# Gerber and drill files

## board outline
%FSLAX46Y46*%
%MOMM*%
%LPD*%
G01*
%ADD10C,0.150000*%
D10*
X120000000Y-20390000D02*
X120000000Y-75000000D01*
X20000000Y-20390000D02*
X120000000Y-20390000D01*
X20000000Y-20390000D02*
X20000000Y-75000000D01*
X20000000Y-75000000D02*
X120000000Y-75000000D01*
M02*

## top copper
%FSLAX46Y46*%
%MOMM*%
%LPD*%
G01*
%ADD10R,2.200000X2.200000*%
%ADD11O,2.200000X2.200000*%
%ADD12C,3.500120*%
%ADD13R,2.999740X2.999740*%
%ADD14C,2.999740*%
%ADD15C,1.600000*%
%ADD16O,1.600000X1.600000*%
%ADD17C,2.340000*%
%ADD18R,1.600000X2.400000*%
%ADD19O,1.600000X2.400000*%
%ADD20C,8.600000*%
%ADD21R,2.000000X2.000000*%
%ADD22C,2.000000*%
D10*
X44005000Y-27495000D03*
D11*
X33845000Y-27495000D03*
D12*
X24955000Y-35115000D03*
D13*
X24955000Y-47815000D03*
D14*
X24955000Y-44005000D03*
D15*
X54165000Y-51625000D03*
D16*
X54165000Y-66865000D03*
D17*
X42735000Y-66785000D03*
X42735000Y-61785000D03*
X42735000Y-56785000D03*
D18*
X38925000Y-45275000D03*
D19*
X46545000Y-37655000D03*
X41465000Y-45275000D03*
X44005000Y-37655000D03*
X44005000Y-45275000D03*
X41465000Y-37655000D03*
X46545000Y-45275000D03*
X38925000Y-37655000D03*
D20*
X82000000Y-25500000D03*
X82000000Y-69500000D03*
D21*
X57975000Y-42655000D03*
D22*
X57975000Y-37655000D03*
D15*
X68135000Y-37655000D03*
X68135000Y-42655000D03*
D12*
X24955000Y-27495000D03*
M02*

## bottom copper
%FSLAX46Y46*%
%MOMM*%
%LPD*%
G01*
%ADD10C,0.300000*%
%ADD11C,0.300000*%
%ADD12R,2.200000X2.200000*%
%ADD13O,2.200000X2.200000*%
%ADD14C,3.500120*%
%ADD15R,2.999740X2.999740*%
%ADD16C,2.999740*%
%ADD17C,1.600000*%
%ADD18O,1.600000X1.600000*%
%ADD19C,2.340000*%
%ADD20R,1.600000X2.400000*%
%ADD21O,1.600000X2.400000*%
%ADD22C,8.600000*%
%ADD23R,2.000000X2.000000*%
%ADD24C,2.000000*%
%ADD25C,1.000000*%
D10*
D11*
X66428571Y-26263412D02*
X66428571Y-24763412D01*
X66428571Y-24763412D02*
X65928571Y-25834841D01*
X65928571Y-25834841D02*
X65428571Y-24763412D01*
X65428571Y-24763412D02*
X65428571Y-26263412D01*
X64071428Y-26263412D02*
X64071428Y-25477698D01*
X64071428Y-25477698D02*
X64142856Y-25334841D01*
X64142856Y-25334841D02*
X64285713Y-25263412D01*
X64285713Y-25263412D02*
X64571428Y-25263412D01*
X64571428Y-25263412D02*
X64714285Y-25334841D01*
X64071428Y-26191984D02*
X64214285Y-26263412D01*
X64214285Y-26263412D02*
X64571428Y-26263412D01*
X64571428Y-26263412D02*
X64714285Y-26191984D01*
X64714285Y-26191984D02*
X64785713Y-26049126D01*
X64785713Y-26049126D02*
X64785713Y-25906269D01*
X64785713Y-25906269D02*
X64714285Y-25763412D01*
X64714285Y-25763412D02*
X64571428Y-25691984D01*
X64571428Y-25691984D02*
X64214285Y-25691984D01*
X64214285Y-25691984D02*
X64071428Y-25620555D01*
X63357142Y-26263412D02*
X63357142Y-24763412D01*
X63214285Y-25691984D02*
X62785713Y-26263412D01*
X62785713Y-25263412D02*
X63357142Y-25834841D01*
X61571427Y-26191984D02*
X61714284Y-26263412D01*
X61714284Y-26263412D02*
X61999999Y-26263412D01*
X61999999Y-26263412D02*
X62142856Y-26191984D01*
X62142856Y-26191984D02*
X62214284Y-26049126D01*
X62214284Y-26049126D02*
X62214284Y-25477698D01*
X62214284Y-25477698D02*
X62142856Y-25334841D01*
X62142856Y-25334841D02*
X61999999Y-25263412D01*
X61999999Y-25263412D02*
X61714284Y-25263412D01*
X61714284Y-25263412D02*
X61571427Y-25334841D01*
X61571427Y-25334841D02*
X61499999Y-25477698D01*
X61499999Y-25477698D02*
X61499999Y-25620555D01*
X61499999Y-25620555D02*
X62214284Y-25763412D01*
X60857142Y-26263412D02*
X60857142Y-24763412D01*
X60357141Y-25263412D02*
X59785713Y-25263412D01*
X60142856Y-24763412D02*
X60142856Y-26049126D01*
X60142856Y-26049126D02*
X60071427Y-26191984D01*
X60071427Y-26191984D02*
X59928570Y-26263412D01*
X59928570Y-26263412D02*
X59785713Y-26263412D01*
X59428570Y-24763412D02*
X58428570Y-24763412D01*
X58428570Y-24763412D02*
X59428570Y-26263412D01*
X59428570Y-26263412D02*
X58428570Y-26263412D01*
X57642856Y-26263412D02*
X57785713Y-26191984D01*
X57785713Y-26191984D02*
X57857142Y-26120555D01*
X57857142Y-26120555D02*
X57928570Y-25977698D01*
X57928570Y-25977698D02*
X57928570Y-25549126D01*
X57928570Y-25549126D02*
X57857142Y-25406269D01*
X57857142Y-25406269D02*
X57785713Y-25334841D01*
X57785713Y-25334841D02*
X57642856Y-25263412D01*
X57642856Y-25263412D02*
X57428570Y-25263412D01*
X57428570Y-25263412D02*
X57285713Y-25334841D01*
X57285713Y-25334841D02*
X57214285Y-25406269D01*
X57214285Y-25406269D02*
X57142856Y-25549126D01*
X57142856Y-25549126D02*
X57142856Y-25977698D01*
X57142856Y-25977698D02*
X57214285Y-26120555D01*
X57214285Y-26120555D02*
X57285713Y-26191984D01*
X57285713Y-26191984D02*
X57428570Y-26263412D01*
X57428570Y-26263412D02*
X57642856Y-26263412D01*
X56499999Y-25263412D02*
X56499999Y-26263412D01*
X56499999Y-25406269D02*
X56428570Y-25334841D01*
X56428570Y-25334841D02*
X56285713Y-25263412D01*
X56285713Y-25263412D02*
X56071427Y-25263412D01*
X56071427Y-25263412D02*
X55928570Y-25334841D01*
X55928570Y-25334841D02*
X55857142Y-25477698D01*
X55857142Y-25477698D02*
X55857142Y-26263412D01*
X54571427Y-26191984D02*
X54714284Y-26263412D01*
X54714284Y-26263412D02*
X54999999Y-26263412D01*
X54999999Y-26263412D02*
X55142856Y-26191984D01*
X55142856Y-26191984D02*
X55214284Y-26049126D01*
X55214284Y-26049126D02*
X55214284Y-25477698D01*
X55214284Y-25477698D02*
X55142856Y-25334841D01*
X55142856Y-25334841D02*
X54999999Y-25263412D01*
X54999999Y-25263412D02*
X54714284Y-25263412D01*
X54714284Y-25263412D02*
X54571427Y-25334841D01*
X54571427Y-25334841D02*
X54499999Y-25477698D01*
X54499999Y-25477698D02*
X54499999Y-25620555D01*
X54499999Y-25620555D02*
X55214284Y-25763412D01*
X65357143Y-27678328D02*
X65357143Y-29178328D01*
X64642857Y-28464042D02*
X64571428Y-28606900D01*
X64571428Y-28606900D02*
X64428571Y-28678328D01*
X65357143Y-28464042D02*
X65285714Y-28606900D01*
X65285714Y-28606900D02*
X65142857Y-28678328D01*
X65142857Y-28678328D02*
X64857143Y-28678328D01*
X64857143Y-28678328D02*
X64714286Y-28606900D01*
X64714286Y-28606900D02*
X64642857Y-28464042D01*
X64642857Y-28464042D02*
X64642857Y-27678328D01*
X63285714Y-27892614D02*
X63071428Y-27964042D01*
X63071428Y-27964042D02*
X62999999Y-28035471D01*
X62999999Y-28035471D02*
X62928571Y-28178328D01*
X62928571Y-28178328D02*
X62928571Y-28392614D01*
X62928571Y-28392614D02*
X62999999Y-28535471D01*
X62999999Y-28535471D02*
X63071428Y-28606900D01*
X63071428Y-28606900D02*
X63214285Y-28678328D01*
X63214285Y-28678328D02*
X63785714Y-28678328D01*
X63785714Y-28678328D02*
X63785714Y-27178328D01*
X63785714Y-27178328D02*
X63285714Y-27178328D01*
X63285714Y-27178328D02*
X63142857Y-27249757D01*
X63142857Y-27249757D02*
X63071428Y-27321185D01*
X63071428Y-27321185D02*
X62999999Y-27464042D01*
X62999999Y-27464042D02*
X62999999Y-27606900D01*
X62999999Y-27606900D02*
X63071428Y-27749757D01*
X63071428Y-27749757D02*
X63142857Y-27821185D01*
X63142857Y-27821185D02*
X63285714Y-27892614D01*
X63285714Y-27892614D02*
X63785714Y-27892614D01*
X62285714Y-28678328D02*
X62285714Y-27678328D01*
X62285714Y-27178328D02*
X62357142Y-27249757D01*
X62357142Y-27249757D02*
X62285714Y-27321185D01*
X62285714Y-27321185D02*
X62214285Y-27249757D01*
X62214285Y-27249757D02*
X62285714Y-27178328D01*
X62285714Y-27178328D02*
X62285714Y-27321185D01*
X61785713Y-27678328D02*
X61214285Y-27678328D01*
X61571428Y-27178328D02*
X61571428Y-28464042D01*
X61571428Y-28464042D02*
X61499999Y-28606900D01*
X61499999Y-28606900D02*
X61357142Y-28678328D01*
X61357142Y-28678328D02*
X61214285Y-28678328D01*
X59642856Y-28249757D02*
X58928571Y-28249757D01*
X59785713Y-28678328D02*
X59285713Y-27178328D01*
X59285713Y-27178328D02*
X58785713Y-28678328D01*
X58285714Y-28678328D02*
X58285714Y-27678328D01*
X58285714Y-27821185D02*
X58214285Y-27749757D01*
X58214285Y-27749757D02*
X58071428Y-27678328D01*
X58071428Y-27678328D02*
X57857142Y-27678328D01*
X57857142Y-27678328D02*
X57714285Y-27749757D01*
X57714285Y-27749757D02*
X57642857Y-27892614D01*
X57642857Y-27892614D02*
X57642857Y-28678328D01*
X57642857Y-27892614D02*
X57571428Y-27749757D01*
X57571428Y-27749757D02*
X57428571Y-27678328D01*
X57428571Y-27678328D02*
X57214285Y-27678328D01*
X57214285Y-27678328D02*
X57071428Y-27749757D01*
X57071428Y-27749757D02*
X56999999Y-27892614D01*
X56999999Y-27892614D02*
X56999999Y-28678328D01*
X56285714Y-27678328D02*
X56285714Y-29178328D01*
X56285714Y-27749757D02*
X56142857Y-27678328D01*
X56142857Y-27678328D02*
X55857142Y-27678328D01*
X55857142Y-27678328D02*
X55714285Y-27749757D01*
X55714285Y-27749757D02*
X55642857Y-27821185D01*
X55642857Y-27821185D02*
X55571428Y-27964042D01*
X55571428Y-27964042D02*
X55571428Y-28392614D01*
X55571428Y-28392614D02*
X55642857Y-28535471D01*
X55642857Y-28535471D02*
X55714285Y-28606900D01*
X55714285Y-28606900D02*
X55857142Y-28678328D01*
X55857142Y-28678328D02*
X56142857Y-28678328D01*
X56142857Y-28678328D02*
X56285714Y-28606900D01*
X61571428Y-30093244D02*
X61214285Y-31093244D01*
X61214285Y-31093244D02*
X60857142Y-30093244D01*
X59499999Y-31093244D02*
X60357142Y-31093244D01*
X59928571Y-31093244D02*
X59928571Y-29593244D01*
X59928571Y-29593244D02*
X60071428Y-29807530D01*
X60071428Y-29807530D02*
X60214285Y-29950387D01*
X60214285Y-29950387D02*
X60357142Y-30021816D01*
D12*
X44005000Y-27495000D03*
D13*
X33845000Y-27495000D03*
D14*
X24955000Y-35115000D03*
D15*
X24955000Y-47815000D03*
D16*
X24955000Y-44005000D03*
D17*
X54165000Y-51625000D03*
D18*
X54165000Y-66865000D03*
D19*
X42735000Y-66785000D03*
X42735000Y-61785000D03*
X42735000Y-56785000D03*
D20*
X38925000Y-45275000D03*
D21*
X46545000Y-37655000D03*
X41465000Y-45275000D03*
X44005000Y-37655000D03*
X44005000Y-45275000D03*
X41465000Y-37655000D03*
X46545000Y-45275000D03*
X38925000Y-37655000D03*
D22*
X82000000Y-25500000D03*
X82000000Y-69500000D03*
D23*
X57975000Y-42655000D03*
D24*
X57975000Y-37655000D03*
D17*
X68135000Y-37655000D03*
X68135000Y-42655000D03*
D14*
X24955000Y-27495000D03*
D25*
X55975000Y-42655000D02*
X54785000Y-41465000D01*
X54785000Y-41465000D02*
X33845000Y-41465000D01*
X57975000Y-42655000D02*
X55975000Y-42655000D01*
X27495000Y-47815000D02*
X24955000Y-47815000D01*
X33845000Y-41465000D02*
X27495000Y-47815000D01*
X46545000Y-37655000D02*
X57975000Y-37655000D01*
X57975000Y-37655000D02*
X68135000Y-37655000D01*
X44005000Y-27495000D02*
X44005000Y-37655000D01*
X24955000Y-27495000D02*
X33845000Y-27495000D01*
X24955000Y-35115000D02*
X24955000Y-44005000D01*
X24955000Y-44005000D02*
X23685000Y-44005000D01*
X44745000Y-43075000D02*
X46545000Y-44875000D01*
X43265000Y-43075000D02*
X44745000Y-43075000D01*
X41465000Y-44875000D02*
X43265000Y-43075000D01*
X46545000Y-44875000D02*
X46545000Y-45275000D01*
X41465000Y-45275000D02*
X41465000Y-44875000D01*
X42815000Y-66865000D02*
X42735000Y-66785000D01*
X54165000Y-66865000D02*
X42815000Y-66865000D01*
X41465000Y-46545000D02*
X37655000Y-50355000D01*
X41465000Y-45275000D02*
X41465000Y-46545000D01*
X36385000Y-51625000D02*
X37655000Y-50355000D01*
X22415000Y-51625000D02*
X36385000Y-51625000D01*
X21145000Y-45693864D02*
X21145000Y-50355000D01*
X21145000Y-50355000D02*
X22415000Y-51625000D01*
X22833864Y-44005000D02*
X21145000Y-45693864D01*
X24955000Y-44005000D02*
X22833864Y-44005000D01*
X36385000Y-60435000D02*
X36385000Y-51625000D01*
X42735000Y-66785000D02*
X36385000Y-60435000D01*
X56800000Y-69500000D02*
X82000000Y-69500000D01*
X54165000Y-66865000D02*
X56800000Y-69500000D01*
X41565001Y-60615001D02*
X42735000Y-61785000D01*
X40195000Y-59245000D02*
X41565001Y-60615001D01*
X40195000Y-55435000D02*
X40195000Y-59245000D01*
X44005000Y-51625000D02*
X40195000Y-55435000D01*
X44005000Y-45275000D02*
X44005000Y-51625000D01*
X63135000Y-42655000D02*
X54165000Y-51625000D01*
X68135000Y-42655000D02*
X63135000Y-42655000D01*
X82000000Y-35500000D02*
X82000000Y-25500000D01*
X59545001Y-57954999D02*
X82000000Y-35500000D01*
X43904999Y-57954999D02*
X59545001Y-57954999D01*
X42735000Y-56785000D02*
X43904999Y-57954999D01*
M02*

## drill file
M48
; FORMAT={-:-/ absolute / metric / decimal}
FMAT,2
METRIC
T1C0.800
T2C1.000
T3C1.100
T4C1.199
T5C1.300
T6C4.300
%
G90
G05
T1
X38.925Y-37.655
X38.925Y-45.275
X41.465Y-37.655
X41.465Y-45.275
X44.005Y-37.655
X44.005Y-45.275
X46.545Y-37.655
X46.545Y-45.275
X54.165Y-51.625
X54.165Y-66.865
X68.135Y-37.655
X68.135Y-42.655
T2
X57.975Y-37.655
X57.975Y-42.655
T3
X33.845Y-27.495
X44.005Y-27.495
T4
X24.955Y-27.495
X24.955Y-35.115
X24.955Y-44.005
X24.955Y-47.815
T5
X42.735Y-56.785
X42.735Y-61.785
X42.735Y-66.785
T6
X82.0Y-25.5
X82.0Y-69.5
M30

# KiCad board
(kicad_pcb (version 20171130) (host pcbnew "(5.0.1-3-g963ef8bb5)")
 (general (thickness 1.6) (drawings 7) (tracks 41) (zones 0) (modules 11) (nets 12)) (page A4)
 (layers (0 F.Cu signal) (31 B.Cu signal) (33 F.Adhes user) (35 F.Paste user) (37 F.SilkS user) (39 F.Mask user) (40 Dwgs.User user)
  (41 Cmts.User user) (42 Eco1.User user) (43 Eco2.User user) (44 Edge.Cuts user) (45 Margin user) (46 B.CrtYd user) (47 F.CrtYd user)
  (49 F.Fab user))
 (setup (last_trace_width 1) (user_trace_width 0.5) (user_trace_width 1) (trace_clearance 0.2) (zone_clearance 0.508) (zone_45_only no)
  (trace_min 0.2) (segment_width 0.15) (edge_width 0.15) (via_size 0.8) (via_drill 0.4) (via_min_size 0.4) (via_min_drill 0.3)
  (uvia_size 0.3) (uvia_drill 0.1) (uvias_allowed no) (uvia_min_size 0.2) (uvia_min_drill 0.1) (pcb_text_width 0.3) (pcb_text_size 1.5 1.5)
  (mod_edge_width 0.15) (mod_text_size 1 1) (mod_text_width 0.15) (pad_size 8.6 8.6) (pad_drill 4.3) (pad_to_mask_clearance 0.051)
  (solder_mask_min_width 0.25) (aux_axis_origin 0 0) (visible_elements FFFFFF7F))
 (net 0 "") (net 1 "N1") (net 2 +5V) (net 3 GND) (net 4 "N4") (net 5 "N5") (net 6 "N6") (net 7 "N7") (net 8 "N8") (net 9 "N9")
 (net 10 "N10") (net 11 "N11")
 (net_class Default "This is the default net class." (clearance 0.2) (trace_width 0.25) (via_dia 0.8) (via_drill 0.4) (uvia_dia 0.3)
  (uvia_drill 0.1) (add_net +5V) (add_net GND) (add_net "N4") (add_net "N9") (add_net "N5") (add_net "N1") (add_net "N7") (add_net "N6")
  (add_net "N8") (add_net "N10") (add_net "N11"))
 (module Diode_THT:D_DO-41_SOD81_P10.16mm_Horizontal (layer F.Cu) (at 44.005 27.495 180)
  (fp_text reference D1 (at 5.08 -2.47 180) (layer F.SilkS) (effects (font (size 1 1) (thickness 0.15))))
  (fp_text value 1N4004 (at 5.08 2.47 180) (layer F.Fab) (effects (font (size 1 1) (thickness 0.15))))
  (pad 1 thru_hole rect (at 0 0 180) (size 2.2 2.2) (drill 1.1) (layers *.Cu *.Mask) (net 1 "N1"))
  (pad 2 thru_hole oval (at 10.16 0 180) (size 2.2 2.2) (drill 1.1) (layers *.Cu *.Mask) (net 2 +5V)))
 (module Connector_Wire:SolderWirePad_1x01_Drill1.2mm (layer F.Cu) (at 24.955 35.115)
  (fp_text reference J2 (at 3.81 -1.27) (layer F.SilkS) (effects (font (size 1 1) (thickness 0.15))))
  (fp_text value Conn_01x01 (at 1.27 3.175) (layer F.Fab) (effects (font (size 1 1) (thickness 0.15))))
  (pad 1 thru_hole circle (at 0 0) (size 3.50012 3.50012) (drill 1.19888) (layers *.Cu *.Mask) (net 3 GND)))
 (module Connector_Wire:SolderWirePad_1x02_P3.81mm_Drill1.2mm (layer F.Cu) (at 24.955 47.815 90)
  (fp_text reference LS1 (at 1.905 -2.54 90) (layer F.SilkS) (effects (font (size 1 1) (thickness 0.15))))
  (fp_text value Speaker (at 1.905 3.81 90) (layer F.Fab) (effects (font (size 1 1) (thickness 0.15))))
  (pad 1 thru_hole rect (at 0 0 90) (size 2.99974 2.99974) (drill 1.19888) (layers *.Cu *.Mask) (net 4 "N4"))
  (pad 2 thru_hole circle (at 3.81 0 90) (size 2.99974 2.99974) (drill 1.19888) (layers *.Cu *.Mask) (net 3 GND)))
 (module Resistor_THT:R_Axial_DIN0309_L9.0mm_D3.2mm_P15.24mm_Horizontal (layer F.Cu) (at 54.165 51.625 270)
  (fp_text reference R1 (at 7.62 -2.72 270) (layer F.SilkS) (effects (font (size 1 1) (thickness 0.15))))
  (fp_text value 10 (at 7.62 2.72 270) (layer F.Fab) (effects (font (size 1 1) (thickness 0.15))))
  (pad 1 thru_hole circle (at 0 0 270) (size 1.6 1.6) (drill 0.8) (layers *.Cu *.Mask) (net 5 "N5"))
  (pad 2 thru_hole oval (at 15.24 0 270) (size 1.6 1.6) (drill 0.8) (layers *.Cu *.Mask) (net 3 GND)))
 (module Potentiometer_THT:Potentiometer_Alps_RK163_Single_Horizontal (layer F.Cu) (at 42.735 56.785 180)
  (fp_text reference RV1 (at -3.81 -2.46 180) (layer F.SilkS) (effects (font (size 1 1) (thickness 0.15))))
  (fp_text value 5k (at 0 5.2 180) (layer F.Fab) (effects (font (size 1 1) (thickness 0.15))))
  (pad 3 thru_hole circle (at 0 -10 180) (size 2.34 2.34) (drill 1.3) (layers *.Cu *.Mask) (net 3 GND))
  (pad 2 thru_hole circle (at 0 -5 180) (size 2.34 2.34) (drill 1.3) (layers *.Cu *.Mask) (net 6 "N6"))
  (pad 1 thru_hole circle (at 0 0 180) (size 2.34 2.34) (drill 1.3) (layers *.Cu *.Mask) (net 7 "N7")))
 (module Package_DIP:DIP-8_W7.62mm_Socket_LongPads (layer F.Cu) (at 38.925 45.275 90)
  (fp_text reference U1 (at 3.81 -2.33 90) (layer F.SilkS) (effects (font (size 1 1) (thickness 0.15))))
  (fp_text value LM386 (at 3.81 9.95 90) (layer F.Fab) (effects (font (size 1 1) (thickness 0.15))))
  (pad 1 thru_hole rect (at 0 0 90) (size 2.4 1.6) (drill 0.8) (layers *.Cu *.Mask) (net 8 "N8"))
  (pad 5 thru_hole oval (at 7.62 7.62 90) (size 2.4 1.6) (drill 0.8) (layers *.Cu *.Mask) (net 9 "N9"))
  (pad 2 thru_hole oval (at 0 2.54 90) (size 2.4 1.6) (drill 0.8) (layers *.Cu *.Mask) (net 3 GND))
  (pad 6 thru_hole oval (at 7.62 5.08 90) (size 2.4 1.6) (drill 0.8) (layers *.Cu *.Mask) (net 1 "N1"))
  (pad 3 thru_hole oval (at 0 5.08 90) (size 2.4 1.6) (drill 0.8) (layers *.Cu *.Mask) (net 6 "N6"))
  (pad 7 thru_hole oval (at 7.62 2.54 90) (size 2.4 1.6) (drill 0.8) (layers *.Cu *.Mask) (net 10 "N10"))
  (pad 4 thru_hole oval (at 0 7.62 90) (size 2.4 1.6) (drill 0.8) (layers *.Cu *.Mask) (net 3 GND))
  (pad 8 thru_hole oval (at 7.62 0 90) (size 2.4 1.6) (drill 0.8) (layers *.Cu *.Mask) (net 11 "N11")))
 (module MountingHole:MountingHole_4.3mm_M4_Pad (layer F.Cu) (at 82 25.5)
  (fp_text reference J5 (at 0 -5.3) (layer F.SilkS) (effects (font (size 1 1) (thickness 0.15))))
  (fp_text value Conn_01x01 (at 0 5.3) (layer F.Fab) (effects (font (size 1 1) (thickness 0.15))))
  (pad 1 thru_hole circle (at 0 0) (size 8.6 8.6) (drill 4.3) (layers *.Cu *.Mask) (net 7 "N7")))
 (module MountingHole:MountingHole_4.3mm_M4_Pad (layer F.Cu) (at 82 69.5)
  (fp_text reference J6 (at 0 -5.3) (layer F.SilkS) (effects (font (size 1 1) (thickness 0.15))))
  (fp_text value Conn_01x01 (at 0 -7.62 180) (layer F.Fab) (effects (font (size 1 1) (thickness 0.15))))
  (pad 1 thru_hole circle (at 0 0) (size 8.6 8.6) (drill 4.3) (layers *.Cu *.Mask) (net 3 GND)))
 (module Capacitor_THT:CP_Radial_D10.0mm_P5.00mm (layer F.Cu) (at 57.975 42.655 90)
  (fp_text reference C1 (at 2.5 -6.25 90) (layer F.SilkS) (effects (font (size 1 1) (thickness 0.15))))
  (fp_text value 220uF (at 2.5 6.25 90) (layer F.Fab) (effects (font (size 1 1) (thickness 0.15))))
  (pad 1 thru_hole rect (at 0 0 90) (size 2 2) (drill 1) (layers *.Cu *.Mask) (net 4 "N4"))
  (pad 2 thru_hole circle (at 5 0 90) (size 2 2) (drill 1) (layers *.Cu *.Mask) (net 9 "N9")))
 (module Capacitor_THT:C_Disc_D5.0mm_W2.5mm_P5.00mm (layer F.Cu) (at 68.135 37.655 270)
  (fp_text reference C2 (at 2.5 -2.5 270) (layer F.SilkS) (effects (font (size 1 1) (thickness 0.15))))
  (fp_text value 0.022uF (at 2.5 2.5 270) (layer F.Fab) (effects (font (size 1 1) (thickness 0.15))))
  (pad 1 thru_hole circle (at 0 0 270) (size 1.6 1.6) (drill 0.8) (layers *.Cu *.Mask) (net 9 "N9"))
  (pad 2 thru_hole circle (at 5 0 270) (size 1.6 1.6) (drill 0.8) (layers *.Cu *.Mask) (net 5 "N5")))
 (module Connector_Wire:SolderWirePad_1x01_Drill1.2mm (layer F.Cu) (at 24.955 27.495)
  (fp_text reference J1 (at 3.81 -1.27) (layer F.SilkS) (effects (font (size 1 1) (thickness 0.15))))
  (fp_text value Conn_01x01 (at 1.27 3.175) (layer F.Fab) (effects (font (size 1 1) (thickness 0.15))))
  (pad 1 thru_hole circle (at 0 0) (size 3.50012 3.50012) (drill 1.19888) (layers *.Cu *.Mask) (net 2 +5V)))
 (gr_line (start 120 20.39) (end 120 75) (layer Edge.Cuts) (width 0.15))
 (gr_line (start 20 20.39) (end 120 20.39) (layer Edge.Cuts) (width 0.15))
 (gr_line (start 20 20.39) (end 20 75) (layer Edge.Cuts) (width 0.15))
 (gr_line (start 20 75) (end 120 75) (layer Edge.Cuts) (width 0.15))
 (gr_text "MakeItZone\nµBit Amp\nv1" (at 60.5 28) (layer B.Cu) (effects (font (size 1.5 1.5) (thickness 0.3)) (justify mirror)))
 (segment (start 55.975 42.655) (end 54.785 41.465) (width 1) (layer B.Cu) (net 4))
 (segment (start 54.785 41.465) (end 33.845 41.465) (width 1) (layer B.Cu) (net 4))
 (segment (start 57.975 42.655) (end 55.975 42.655) (width 1) (layer B.Cu) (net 4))
 (segment (start 27.495 47.815) (end 24.955 47.815) (width 1) (layer B.Cu) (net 4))
 (segment (start 33.845 41.465) (end 27.495 47.815) (width 1) (layer B.Cu) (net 4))
 (segment (start 46.545 37.655) (end 57.975 37.655) (width 1) (layer B.Cu) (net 9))
 (segment (start 57.975 37.655) (end 68.135 37.655) (width 1) (layer B.Cu) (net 9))
 (segment (start 44.005 27.495) (end 44.005 37.655) (width 1) (layer B.Cu) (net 1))
 (segment (start 24.955 27.495) (end 33.845 27.495) (width 1) (layer B.Cu) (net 2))
 (segment (start 24.955 35.115) (end 24.955 44.005) (width 1) (layer B.Cu) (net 3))
 (segment (start 24.955 44.005) (end 23.685 44.005) (width 1) (layer B.Cu) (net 3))
 (segment (start 44.745 43.075) (end 46.545 44.875) (width 1) (layer B.Cu) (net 3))
 (segment (start 43.265 43.075) (end 44.745 43.075) (width 1) (layer B.Cu) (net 3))
 (segment (start 41.465 44.875) (end 43.265 43.075) (width 1) (layer B.Cu) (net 3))
 (segment (start 46.545 44.875) (end 46.545 45.275) (width 1) (layer B.Cu) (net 3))
 (segment (start 41.465 45.275) (end 41.465 44.875) (width 1) (layer B.Cu) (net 3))
 (segment (start 42.815 66.865) (end 42.735 66.785) (width 1) (layer B.Cu) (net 3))
 (segment (start 54.165 66.865) (end 42.815 66.865) (width 1) (layer B.Cu) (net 3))
 (segment (start 41.465 46.545) (end 37.655 50.355) (width 1) (layer B.Cu) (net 3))
 (segment (start 41.465 45.275) (end 41.465 46.545) (width 1) (layer B.Cu) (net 3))
 (segment (start 36.385 51.625) (end 37.655 50.355) (width 1) (layer B.Cu) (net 3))
 (segment (start 22.415 51.625) (end 36.385 51.625) (width 1) (layer B.Cu) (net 3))
 (segment (start 21.145 45.693864) (end 21.145 50.355) (width 1) (layer B.Cu) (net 3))
 (segment (start 21.145 50.355) (end 22.415 51.625) (width 1) (layer B.Cu) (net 3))
 (segment (start 22.833864 44.005) (end 21.145 45.693864) (width 1) (layer B.Cu) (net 3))
 (segment (start 24.955 44.005) (end 22.833864 44.005) (width 1) (layer B.Cu) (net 3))
 (segment (start 36.385 60.435) (end 36.385 51.625) (width 1) (layer B.Cu) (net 3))
 (segment (start 42.735 66.785) (end 36.385 60.435) (width 1) (layer B.Cu) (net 3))
 (segment (start 56.8 69.5) (end 82 69.5) (width 1) (layer B.Cu) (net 3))
 (segment (start 54.165 66.865) (end 56.8 69.5) (width 1) (layer B.Cu) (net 3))
 (segment (start 41.565001 60.615001) (end 42.735 61.785) (width 1) (layer B.Cu) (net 6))
 (segment (start 40.195 59.245) (end 41.565001 60.615001) (width 1) (layer B.Cu) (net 6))
 (segment (start 40.195 55.435) (end 40.195 59.245) (width 1) (layer B.Cu) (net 6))
 (segment (start 44.005 51.625) (end 40.195 55.435) (width 1) (layer B.Cu) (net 6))
 (segment (start 44.005 45.275) (end 44.005 51.625) (width 1) (layer B.Cu) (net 6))
 (segment (start 63.135 42.655) (end 54.165 51.625) (width 1) (layer B.Cu) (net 5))
 (segment (start 68.135 42.655) (end 63.135 42.655) (width 1) (layer B.Cu) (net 5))
 (segment (start 82 35.5) (end 82 25.5) (width 1) (layer B.Cu) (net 7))
 (segment (start 59.545001 57.954999) (end 82 35.5) (width 1) (layer B.Cu) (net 7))
 (segment (start 43.904999 57.954999) (end 59.545001 57.954999) (width 1) (layer B.Cu) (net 7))
 (segment (start 42.735 56.785) (end 43.904999 57.954999) (width 1) (layer B.Cu) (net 7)))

